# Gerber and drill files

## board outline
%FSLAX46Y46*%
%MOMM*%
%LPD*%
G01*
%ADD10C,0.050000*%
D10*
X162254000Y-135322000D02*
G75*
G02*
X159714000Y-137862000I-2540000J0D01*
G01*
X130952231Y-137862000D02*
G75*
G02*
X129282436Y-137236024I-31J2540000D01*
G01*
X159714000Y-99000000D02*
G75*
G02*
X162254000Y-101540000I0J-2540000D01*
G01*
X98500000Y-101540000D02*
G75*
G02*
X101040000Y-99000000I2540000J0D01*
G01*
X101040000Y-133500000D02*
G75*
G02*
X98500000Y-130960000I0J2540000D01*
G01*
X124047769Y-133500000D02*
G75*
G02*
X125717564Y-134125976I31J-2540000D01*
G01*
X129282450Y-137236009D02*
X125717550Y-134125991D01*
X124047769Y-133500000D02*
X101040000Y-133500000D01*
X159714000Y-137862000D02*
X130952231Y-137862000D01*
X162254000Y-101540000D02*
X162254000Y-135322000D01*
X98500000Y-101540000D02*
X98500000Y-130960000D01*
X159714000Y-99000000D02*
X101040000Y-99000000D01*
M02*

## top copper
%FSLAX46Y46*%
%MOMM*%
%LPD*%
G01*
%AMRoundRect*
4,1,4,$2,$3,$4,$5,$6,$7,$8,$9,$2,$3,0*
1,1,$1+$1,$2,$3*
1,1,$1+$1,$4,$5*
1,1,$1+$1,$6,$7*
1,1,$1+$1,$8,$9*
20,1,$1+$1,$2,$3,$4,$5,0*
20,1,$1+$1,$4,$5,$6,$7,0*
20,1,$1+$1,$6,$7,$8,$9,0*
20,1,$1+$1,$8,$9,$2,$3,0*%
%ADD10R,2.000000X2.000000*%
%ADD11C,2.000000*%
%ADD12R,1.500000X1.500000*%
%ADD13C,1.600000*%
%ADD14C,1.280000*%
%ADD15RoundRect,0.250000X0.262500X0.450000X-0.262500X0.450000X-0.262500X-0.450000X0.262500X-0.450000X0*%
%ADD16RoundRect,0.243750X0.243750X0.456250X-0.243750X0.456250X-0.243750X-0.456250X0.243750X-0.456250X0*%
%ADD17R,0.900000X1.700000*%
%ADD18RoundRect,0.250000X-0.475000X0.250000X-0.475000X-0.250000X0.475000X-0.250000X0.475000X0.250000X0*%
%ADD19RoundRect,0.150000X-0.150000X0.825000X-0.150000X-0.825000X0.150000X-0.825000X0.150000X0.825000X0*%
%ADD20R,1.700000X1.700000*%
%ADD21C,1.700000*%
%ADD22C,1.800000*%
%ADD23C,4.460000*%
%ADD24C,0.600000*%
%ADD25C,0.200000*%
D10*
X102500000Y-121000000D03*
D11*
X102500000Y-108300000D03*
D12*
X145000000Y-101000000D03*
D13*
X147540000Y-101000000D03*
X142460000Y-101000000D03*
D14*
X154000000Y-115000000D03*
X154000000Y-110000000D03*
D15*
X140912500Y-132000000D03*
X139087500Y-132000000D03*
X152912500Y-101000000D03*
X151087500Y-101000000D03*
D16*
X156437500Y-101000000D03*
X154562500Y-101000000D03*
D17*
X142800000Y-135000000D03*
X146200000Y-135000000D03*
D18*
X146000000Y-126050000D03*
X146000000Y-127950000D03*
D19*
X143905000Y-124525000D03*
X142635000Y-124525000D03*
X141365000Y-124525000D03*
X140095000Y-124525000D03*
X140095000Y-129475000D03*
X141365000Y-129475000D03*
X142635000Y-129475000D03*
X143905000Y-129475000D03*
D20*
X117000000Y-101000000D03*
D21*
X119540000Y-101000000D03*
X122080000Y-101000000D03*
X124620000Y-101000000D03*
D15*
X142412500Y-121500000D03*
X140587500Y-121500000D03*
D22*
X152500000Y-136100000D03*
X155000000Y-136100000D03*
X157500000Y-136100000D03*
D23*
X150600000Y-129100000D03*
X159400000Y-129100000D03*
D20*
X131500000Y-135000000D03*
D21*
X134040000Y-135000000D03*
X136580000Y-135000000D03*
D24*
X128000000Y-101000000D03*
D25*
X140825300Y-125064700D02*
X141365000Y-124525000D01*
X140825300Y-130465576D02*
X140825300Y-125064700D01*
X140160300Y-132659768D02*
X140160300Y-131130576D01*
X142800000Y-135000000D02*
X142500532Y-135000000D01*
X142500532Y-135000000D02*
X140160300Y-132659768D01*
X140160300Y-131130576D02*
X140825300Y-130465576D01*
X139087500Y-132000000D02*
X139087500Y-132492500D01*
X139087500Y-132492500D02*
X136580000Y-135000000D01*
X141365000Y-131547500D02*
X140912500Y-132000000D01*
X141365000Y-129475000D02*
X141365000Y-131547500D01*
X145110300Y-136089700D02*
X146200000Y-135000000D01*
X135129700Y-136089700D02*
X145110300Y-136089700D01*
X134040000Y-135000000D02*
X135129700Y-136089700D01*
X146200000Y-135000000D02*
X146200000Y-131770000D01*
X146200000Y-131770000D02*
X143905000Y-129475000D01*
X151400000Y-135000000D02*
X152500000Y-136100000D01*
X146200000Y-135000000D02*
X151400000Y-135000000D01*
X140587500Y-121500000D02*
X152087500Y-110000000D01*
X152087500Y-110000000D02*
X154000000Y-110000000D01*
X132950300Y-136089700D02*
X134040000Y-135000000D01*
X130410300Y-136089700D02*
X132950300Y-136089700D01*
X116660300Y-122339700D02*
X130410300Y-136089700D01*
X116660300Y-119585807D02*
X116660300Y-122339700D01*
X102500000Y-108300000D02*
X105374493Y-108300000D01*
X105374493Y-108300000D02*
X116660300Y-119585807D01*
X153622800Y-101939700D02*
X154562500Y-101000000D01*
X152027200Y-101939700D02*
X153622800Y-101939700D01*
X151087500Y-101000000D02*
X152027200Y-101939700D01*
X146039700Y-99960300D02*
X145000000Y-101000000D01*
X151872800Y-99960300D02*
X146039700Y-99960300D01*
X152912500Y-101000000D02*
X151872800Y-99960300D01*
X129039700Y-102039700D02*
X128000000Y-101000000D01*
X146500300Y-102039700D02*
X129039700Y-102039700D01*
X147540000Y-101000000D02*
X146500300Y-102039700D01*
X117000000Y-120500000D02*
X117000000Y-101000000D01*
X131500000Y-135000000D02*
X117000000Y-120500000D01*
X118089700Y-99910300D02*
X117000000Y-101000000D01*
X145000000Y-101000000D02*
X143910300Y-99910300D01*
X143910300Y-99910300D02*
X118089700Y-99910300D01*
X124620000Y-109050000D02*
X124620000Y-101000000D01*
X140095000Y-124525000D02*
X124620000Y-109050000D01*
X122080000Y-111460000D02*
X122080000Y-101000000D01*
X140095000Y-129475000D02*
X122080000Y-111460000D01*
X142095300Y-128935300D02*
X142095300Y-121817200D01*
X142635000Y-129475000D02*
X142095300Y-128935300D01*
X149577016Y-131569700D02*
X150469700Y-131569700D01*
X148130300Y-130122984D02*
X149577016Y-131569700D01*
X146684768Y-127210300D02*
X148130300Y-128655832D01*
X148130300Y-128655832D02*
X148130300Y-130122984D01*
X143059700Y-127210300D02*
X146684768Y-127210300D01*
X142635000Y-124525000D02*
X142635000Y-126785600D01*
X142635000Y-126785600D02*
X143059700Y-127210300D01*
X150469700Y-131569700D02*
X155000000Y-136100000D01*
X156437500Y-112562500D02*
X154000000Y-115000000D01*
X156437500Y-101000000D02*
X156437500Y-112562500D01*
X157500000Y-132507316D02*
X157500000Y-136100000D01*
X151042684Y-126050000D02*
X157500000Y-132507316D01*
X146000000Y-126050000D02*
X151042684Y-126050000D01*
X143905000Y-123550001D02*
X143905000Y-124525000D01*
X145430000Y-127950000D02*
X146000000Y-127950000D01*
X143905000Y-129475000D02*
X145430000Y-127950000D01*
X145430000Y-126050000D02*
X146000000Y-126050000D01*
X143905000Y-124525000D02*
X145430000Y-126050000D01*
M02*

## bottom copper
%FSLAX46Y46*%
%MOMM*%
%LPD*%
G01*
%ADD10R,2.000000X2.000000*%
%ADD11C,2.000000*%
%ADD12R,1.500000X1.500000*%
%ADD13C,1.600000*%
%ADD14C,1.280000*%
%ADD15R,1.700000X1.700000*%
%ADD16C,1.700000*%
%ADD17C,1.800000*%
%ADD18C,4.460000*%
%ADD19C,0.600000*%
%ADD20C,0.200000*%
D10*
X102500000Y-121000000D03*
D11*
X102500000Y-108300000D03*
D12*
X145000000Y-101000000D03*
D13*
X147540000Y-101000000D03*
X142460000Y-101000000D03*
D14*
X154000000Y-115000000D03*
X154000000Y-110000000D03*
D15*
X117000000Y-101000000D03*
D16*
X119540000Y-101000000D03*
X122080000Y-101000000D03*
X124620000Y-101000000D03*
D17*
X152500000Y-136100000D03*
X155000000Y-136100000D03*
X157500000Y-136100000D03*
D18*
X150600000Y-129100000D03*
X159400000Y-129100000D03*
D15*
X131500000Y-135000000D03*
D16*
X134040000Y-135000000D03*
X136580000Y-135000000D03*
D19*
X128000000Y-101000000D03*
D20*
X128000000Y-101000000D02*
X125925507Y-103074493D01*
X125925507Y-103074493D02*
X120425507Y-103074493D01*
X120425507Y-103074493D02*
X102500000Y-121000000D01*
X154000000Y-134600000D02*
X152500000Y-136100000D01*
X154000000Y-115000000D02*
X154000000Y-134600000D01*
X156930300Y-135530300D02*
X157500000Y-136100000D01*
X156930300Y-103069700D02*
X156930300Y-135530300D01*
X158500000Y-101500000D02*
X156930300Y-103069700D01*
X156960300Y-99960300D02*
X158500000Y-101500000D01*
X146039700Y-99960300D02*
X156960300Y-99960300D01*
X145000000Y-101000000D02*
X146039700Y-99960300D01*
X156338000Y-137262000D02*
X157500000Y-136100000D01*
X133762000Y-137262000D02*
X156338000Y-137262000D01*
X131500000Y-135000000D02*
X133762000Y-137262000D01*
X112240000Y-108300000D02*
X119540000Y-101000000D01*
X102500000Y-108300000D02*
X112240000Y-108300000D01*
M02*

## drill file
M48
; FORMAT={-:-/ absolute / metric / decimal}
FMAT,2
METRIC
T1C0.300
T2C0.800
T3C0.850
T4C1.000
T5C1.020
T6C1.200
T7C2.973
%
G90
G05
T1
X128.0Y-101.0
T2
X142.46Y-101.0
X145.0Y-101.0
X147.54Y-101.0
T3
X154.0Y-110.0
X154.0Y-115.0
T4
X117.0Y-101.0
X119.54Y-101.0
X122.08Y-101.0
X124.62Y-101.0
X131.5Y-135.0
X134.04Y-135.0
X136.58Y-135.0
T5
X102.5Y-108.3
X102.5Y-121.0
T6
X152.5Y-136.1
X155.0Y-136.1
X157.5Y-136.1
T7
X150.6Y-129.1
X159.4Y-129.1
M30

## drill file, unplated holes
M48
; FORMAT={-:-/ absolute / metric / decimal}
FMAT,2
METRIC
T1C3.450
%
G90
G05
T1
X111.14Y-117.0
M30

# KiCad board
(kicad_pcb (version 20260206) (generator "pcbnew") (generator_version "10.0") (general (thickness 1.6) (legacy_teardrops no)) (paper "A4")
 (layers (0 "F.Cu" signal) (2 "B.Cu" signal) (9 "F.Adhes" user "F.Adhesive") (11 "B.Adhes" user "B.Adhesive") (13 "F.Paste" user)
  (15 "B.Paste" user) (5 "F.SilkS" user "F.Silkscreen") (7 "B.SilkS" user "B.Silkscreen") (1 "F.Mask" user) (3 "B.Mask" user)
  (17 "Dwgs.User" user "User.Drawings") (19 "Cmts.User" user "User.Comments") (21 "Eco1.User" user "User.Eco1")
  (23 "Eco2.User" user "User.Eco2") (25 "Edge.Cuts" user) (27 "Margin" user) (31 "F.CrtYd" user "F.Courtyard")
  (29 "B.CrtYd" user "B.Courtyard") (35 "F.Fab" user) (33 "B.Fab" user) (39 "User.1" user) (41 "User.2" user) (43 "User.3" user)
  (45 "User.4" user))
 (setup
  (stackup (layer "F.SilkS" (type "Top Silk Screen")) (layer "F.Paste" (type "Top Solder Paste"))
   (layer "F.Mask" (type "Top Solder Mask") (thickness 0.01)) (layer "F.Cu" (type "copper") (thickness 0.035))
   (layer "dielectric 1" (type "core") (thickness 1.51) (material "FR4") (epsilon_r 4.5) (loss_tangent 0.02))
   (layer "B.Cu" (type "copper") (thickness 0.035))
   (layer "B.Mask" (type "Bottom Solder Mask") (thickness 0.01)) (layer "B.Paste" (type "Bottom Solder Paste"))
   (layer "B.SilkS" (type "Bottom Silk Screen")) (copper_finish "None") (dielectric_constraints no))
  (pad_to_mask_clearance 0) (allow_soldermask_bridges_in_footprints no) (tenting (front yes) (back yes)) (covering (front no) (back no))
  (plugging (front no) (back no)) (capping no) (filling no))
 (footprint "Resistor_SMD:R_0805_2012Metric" (layer "F.Cu") (at 140 132 180)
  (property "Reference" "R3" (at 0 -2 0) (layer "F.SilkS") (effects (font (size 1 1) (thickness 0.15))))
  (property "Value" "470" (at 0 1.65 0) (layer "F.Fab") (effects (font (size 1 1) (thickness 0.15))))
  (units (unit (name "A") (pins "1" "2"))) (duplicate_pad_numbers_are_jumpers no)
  (pad "1" smd roundrect (at -0.9125 0 180) (size 1.025 1.4) (layers "F.Cu" "F.Mask" "F.Paste") (roundrect_rratio 0.243902)
   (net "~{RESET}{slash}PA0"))
  (pad "2" smd roundrect (at 0.9125 0 180) (size 1.025 1.4) (layers "F.Cu" "F.Mask" "F.Paste") (roundrect_rratio 0.243902) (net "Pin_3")))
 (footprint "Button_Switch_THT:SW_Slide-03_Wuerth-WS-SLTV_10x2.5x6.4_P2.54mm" (layer "F.Cu") (at 145 101 180)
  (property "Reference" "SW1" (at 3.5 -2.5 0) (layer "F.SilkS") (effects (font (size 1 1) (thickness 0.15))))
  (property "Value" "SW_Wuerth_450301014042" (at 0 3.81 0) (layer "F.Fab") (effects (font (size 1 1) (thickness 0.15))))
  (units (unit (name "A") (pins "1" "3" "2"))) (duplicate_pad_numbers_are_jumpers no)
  (pad "1" thru_hole rect (at 0 0 180) (size 1.5 1.5) (drill 0.8) (layers "*.Cu" "*.Mask") (remove_unused_layers no) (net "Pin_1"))
  (pad "2" thru_hole circle (at -2.54 0 180) (size 1.6 1.6) (drill 0.8) (layers "*.Cu" "*.Mask") (remove_unused_layers no)
   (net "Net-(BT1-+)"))
  (pad "3" thru_hole circle (at 2.54 0 180) (size 1.6 1.6) (drill 0.8) (layers "*.Cu" "*.Mask") (remove_unused_layers no)
   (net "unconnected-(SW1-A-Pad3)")))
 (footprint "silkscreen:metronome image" (layer "F.Cu") (at 143.5 113)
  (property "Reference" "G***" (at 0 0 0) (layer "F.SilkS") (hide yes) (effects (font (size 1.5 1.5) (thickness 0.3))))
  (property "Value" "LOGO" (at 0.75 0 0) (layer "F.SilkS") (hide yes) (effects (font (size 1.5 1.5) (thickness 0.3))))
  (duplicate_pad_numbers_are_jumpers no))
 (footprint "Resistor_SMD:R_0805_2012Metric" (layer "F.Cu") (at 152 101 180)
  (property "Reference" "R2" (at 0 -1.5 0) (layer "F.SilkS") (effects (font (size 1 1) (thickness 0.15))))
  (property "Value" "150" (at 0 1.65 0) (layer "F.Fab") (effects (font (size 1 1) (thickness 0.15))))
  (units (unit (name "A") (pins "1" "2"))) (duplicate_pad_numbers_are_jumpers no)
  (pad "1" smd roundrect (at -0.9125 0 180) (size 1.025 1.4) (layers "F.Cu" "F.Mask" "F.Paste") (roundrect_rratio 0.243902) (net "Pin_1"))
  (pad "2" smd roundrect (at 0.9125 0 180) (size 1.025 1.4) (layers "F.Cu" "F.Mask" "F.Paste") (roundrect_rratio 0.243902)
   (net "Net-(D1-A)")))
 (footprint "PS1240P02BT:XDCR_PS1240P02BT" (layer "F.Cu") (at 154 112.5 -90)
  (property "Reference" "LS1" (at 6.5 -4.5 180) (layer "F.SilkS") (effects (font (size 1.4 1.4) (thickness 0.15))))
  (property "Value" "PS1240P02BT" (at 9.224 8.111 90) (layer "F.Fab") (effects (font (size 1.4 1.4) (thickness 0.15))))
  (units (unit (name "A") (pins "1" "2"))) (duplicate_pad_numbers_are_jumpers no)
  (pad "1" thru_hole circle (at -2.5 0 270) (size 1.28 1.28) (drill 0.85) (layers "*.Cu" "*.Mask") (remove_unused_layers no)
   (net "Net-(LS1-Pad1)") (solder_mask_margin 0.102))
  (pad "2" thru_hole circle (at 2.5 0 270) (size 1.28 1.28) (drill 0.85) (layers "*.Cu" "*.Mask") (remove_unused_layers no) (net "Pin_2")
   (solder_mask_margin 0.102)))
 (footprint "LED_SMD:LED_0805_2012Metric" (layer "F.Cu") (at 155.5 101 180)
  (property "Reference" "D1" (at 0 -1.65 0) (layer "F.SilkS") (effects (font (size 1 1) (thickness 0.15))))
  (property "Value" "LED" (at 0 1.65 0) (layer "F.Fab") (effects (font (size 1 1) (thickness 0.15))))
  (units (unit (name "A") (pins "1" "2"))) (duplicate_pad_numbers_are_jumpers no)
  (pad "1" smd roundrect (at -0.9375 0 180) (size 0.975 1.4) (layers "F.Cu" "F.Mask" "F.Paste") (roundrect_rratio 0.25) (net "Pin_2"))
  (pad "2" smd roundrect (at 0.9375 0 180) (size 0.975 1.4) (layers "F.Cu" "F.Mask" "F.Paste") (roundrect_rratio 0.25) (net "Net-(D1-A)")))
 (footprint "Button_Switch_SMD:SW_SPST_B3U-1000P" (layer "F.Cu") (at 144.5 135)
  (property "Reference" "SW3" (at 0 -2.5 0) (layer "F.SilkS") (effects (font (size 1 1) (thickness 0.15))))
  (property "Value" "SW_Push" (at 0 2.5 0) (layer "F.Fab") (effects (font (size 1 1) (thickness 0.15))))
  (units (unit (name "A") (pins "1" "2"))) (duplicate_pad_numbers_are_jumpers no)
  (pad "1" smd rect (at -1.7 0) (size 0.9 1.7) (layers "F.Cu" "F.Mask" "F.Paste") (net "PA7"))
  (pad "2" smd rect (at 1.7 0) (size 0.9 1.7) (layers "F.Cu" "F.Mask" "F.Paste") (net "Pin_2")))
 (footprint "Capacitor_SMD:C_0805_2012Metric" (layer "F.Cu") (at 146 127 -90)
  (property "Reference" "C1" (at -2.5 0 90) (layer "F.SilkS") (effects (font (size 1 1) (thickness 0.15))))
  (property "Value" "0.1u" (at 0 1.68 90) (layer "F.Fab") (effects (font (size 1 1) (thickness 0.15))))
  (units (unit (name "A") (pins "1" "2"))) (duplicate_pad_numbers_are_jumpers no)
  (pad "1" smd roundrect (at -0.95 0 270) (size 1 1.45) (layers "F.Cu" "F.Mask" "F.Paste") (roundrect_rratio 0.25) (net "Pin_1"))
  (pad "2" smd roundrect (at 0.95 0 270) (size 1 1.45) (layers "F.Cu" "F.Mask" "F.Paste") (roundrect_rratio 0.25) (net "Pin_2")))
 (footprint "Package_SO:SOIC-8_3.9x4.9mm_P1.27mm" (layer "F.Cu") (at 142 127 -90)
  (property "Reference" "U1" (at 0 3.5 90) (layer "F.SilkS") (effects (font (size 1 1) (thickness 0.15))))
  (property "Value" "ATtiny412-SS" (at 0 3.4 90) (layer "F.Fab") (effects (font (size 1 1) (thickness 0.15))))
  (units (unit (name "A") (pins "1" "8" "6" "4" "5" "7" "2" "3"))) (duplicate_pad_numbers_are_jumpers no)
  (pad "1" smd roundrect (at -2.475 -1.905 270) (size 1.95 0.6) (layers "F.Cu" "F.Mask" "F.Paste") (roundrect_rratio 0.25) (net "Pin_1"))
  (pad "2" smd roundrect (at -2.475 -0.635 270) (size 1.95 0.6) (layers "F.Cu" "F.Mask" "F.Paste") (roundrect_rratio 0.25) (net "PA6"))
  (pad "3" smd roundrect (at -2.475 0.635 270) (size 1.95 0.6) (layers "F.Cu" "F.Mask" "F.Paste") (roundrect_rratio 0.25) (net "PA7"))
  (pad "4" smd roundrect (at -2.475 1.905 270) (size 1.95 0.6) (layers "F.Cu" "F.Mask" "F.Paste") (roundrect_rratio 0.25) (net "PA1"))
  (pad "5" smd roundrect (at 2.475 1.905 270) (size 1.95 0.6) (layers "F.Cu" "F.Mask" "F.Paste") (roundrect_rratio 0.25) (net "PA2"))
  (pad "6" smd roundrect (at 2.475 0.635 270) (size 1.95 0.6) (layers "F.Cu" "F.Mask" "F.Paste") (roundrect_rratio 0.25)
   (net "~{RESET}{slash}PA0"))
  (pad "7" smd roundrect (at 2.475 -0.635 270) (size 1.95 0.6) (layers "F.Cu" "F.Mask" "F.Paste") (roundrect_rratio 0.25) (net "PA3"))
  (pad "8" smd roundrect (at 2.475 -1.905 270) (size 1.95 0.6) (layers "F.Cu" "F.Mask" "F.Paste") (roundrect_rratio 0.25) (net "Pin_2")))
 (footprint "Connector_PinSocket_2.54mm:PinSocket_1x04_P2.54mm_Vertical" (layer "F.Cu") (at 117 101 90)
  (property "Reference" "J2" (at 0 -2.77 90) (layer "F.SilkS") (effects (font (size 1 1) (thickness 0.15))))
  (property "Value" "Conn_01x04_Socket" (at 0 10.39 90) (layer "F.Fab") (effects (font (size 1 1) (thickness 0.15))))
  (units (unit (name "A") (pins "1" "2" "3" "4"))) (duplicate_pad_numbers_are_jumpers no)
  (pad "1" thru_hole rect (at 0 0 90) (size 1.7 1.7) (drill 1) (layers "*.Cu" "*.Mask") (remove_unused_layers no) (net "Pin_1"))
  (pad "2" thru_hole circle (at 0 2.54 90) (size 1.7 1.7) (drill 1) (layers "*.Cu" "*.Mask") (remove_unused_layers no) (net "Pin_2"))
  (pad "3" thru_hole circle (at 0 5.08 90) (size 1.7 1.7) (drill 1) (layers "*.Cu" "*.Mask") (remove_unused_layers no) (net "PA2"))
  (pad "4" thru_hole circle (at 0 7.62 90) (size 1.7 1.7) (drill 1) (layers "*.Cu" "*.Mask") (remove_unused_layers no) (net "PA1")))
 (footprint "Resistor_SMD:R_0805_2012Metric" (layer "F.Cu") (at 141.5 121.5 180)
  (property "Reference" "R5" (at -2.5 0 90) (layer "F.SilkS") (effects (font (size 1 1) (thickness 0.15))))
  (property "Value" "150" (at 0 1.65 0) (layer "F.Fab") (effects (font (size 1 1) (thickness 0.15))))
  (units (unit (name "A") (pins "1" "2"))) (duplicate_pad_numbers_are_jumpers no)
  (pad "1" smd roundrect (at -0.9125 0 180) (size 1.025 1.4) (layers "F.Cu" "F.Mask" "F.Paste") (roundrect_rratio 0.243902) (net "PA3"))
  (pad "2" smd roundrect (at 0.9125 0 180) (size 1.025 1.4) (layers "F.Cu" "F.Mask" "F.Paste") (roundrect_rratio 0.243902)
   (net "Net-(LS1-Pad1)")))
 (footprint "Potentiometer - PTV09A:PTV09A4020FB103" (layer "F.Cu") (at 155 130.5)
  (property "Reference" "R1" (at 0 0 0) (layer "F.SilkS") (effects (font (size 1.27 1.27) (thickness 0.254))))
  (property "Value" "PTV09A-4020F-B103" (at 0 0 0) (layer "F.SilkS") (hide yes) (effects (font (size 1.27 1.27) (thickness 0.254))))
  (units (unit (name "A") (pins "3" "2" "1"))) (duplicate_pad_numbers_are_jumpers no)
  (pad "1" thru_hole circle (at -2.5 5.6) (size 1.8 1.8) (drill 1.2) (layers "*.Cu" "*.Mask") (remove_unused_layers no) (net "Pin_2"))
  (pad "2" thru_hole circle (at 0 5.6) (size 1.8 1.8) (drill 1.2) (layers "*.Cu" "*.Mask") (remove_unused_layers no) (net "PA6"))
  (pad "3" thru_hole circle (at 2.5 5.6) (size 1.8 1.8) (drill 1.2) (layers "*.Cu" "*.Mask") (remove_unused_layers no) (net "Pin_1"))
  (pad "4" thru_hole circle (at -4.4 -1.4) (size 4.46 4.46) (drill 2.9732) (layers "*.Cu" "*.Mask") (remove_unused_layers no))
  (pad "5" thru_hole circle (at 4.4 -1.4) (size 4.46 4.46) (drill 2.9732) (layers "*.Cu" "*.Mask") (remove_unused_layers no)))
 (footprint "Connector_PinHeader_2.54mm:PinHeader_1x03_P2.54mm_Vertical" (layer "F.Cu") (at 131.5 135 90)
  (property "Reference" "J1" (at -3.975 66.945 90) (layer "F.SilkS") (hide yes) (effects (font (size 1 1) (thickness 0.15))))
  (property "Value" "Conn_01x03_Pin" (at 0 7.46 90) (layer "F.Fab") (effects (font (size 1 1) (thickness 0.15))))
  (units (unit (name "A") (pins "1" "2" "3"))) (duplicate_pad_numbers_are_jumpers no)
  (pad "1" thru_hole rect (at 0 0 90) (size 1.7 1.7) (drill 1) (layers "*.Cu" "*.Mask") (remove_unused_layers no) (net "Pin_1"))
  (pad "2" thru_hole circle (at 0 2.54 90) (size 1.7 1.7) (drill 1) (layers "*.Cu" "*.Mask") (remove_unused_layers no) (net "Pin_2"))
  (pad "3" thru_hole circle (at 0 5.08 90) (size 1.7 1.7) (drill 1) (layers "*.Cu" "*.Mask") (remove_unused_layers no) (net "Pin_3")))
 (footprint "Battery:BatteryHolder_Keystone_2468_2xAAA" (layer "B.Cu") (at 102.5 121)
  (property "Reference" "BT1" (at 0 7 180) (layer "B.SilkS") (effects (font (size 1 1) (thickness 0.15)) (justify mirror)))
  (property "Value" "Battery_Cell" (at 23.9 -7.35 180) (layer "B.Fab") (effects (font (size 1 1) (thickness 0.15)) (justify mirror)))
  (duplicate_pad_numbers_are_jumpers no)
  (pad "" np_thru_hole circle (at 8.64 -4) (size 3.45 3.45) (drill 3.45) (layers "*.Cu"))
  (pad "1" thru_hole rect (at 0 0) (size 2 2) (drill 1.02) (layers "*.Cu" "*.Mask") (remove_unused_layers no) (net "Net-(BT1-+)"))
  (pad "2" thru_hole circle (at 0 -12.7) (size 2 2) (drill 1.02) (layers "*.Cu" "*.Mask") (remove_unused_layers no) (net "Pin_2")))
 (gr_line (start 98.5 101.54) (end 98.5 130.96) (stroke (width 0.05) (type default)) (layer "Edge.Cuts"))
 (gr_arc (start 98.5 101.54) (mid 99.243949 99.743949) (end 101.04 99) (stroke (width 0.05) (type default)) (layer "Edge.Cuts"))
 (gr_arc (start 101.04 133.5) (mid 99.243949 132.756051) (end 98.5 130.96) (stroke (width 0.05) (type default)) (layer "Edge.Cuts"))
 (gr_line (start 124.047769 133.5) (end 101.04 133.5) (stroke (width 0.05) (type default)) (layer "Edge.Cuts"))
 (gr_arc (start 124.047769 133.5) (mid 124.939401 133.661641) (end 125.71755 134.125991) (stroke (width 0.05) (type default))
  (layer "Edge.Cuts"))
 (gr_line (start 129.28245 137.236009) (end 125.71755 134.125991) (stroke (width 0.05) (type default)) (layer "Edge.Cuts"))
 (gr_arc (start 130.952231 137.862) (mid 130.060599 137.700359) (end 129.28245 137.236009) (stroke (width 0.05) (type default))
  (layer "Edge.Cuts"))
 (gr_line (start 159.714 99) (end 101.04 99) (stroke (width 0.05) (type default)) (layer "Edge.Cuts"))
 (gr_arc (start 159.714 99) (mid 161.510051 99.743949) (end 162.254 101.54) (stroke (width 0.05) (type default)) (layer "Edge.Cuts"))
 (gr_line (start 159.714 137.862) (end 130.952231 137.862) (stroke (width 0.05) (type default)) (layer "Edge.Cuts"))
 (gr_line (start 162.254 101.54) (end 162.254 135.322) (stroke (width 0.05) (type default)) (layer "Edge.Cuts"))
 (gr_arc (start 162.254 135.322) (mid 161.510051 137.118051) (end 159.714 137.862) (stroke (width 0.05) (type default)) (layer "Edge.Cuts"))
 (segment (start 141.365 131.5475) (end 140.9125 132) (width 0.2) (layer "F.Cu") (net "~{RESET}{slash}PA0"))
 (segment (start 141.365 129.475) (end 141.365 131.5475) (width 0.2) (layer "F.Cu") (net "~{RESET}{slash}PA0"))
 (segment (start 139.0875 132.4925) (end 136.58 135) (width 0.2) (layer "F.Cu") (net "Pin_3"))
 (segment (start 139.0875 132) (end 139.0875 132.4925) (width 0.2) (layer "F.Cu") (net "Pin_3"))
 (segment (start 146 126.05) (end 151.042684 126.05) (width 0.2) (layer "F.Cu") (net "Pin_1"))
 (segment (start 151.8728 99.9603) (end 146.0397 99.9603) (width 0.2) (layer "F.Cu") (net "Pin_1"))
 (segment (start 143.9103 99.9103) (end 118.0897 99.9103) (width 0.2) (layer "F.Cu") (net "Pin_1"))
 (segment (start 145.43 126.05) (end 146 126.05) (width 0.2) (layer "F.Cu") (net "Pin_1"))
 (segment (start 131.5 135) (end 117 120.5) (width 0.2) (layer "F.Cu") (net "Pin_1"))
 (segment (start 145 101) (end 143.9103 99.9103) (width 0.2) (layer "F.Cu") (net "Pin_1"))
 (segment (start 146.0397 99.9603) (end 145 101) (width 0.2) (layer "F.Cu") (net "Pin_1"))
 (segment (start 151.042684 126.05) (end 157.5 132.507316) (width 0.2) (layer "F.Cu") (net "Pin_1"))
 (segment (start 117 120.5) (end 117 101) (width 0.2) (layer "F.Cu") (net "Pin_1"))
 (segment (start 143.905 124.525) (end 145.43 126.05) (width 0.2) (layer "F.Cu") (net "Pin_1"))
 (segment (start 143.905 123.550001) (end 143.905 124.525) (width 0.2) (layer "F.Cu") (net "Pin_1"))
 (segment (start 118.0897 99.9103) (end 117 101) (width 0.2) (layer "F.Cu") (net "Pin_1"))
 (segment (start 152.9125 101) (end 151.8728 99.9603) (width 0.2) (layer "F.Cu") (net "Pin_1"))
 (segment (start 157.5 132.507316) (end 157.5 136.1) (width 0.2) (layer "F.Cu") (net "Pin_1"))
 (segment (start 133.762 137.262) (end 156.338 137.262) (width 0.2) (layer "B.Cu") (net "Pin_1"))
 (segment (start 156.9303 103.0697) (end 156.9303 135.5303) (width 0.2) (layer "B.Cu") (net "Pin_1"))
 (segment (start 145 101) (end 146.0397 99.9603) (width 0.2) (layer "B.Cu") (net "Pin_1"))
 (segment (start 146.0397 99.9603) (end 156.9603 99.9603) (width 0.2) (layer "B.Cu") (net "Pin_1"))
 (segment (start 158.5 101.5) (end 156.9303 103.0697) (width 0.2) (layer "B.Cu") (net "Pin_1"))
 (segment (start 156.9303 135.5303) (end 157.5 136.1) (width 0.2) (layer "B.Cu") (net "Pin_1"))
 (segment (start 131.5 135) (end 133.762 137.262) (width 0.2) (layer "B.Cu") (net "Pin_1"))
 (segment (start 156.9603 99.9603) (end 158.5 101.5) (width 0.2) (layer "B.Cu") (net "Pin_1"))
 (segment (start 156.338 137.262) (end 157.5 136.1) (width 0.2) (layer "B.Cu") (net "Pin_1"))
 (segment (start 146.5003 102.0397) (end 129.0397 102.0397) (width 0.2) (layer "F.Cu") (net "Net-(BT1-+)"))
 (segment (start 129.0397 102.0397) (end 128 101) (width 0.2) (layer "F.Cu") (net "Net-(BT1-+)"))
 (segment (start 147.54 101) (end 146.5003 102.0397) (width 0.2) (layer "F.Cu") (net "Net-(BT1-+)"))
 (via (at 128 101) (size 0.6) (drill 0.3) (layers "F.Cu" "B.Cu") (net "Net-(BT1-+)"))
 (segment (start 128 101) (end 125.925507 103.074493) (width 0.2) (layer "B.Cu") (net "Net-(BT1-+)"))
 (segment (start 120.425507 103.074493) (end 102.5 121) (width 0.2) (layer "B.Cu") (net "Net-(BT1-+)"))
 (segment (start 125.925507 103.074493) (end 120.425507 103.074493) (width 0.2) (layer "B.Cu") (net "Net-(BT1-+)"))
 (segment (start 153.6228 101.9397) (end 154.5625 101) (width 0.2) (layer "F.Cu") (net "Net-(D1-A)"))
 (segment (start 152.0272 101.9397) (end 153.6228 101.9397) (width 0.2) (layer "F.Cu") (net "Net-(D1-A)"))
 (segment (start 151.0875 101) (end 152.0272 101.9397) (width 0.2) (layer "F.Cu") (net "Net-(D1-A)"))
 (segment (start 152.0875 110) (end 154 110) (width 0.2) (layer "F.Cu") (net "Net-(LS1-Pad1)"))
 (segment (start 140.5875 121.5) (end 152.0875 110) (width 0.2) (layer "F.Cu") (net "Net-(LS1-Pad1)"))
 (segment (start 146.2 131.77) (end 143.905 129.475) (width 0.2) (layer "F.Cu") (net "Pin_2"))
 (segment (start 132.9503 136.0897) (end 134.04 135) (width 0.2) (layer "F.Cu") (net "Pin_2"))
 (segment (start 116.6603 119.585807) (end 116.6603 122.3397) (width 0.2) (layer "F.Cu") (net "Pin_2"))
 (segment (start 135.1297 136.0897) (end 145.1103 136.0897) (width 0.2) (layer "F.Cu") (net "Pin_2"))
 (segment (start 146.2 135) (end 151.4 135) (width 0.2) (layer "F.Cu") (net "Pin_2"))
 (segment (start 145.43 127.95) (end 146 127.95) (width 0.2) (layer "F.Cu") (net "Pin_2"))
 (segment (start 146.2 135) (end 146.2 131.77) (width 0.2) (layer "F.Cu") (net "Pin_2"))
 (segment (start 130.4103 136.0897) (end 132.9503 136.0897) (width 0.2) (layer "F.Cu") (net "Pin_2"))
 (segment (start 156.4375 112.5625) (end 154 115) (width 0.2) (layer "F.Cu") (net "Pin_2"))
 (segment (start 102.5 108.3) (end 105.374493 108.3) (width 0.2) (layer "F.Cu") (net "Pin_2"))
 (segment (start 145.1103 136.0897) (end 146.2 135) (width 0.2) (layer "F.Cu") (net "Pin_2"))
 (segment (start 116.6603 122.3397) (end 130.4103 136.0897) (width 0.2) (layer "F.Cu") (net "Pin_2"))
 (segment (start 105.374493 108.3) (end 116.6603 119.585807) (width 0.2) (layer "F.Cu") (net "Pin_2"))
 (segment (start 156.4375 101) (end 156.4375 112.5625) (width 0.2) (layer "F.Cu") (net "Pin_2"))
 (segment (start 143.905 129.475) (end 145.43 127.95) (width 0.2) (layer "F.Cu") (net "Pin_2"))
 (segment (start 151.4 135) (end 152.5 136.1) (width 0.2) (layer "F.Cu") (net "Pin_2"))
 (segment (start 134.04 135) (end 135.1297 136.0897) (width 0.2) (layer "F.Cu") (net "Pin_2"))
 (segment (start 154 115) (end 154 134.6) (width 0.2) (layer "B.Cu") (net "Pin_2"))
 (segment (start 102.5 108.3) (end 112.24 108.3) (width 0.2) (layer "B.Cu") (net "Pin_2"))
 (segment (start 112.24 108.3) (end 119.54 101) (width 0.2) (layer "B.Cu") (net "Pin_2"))
 (segment (start 154 134.6) (end 152.5 136.1) (width 0.2) (layer "B.Cu") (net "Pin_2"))
 (segment (start 140.8253 125.0647) (end 141.365 124.525) (width 0.2) (layer "F.Cu") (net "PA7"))
 (segment (start 140.8253 130.465576) (end 140.8253 125.0647) (width 0.2) (layer "F.Cu") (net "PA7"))
 (segment (start 140.1603 131.130576) (end 140.8253 130.465576) (width 0.2) (layer "F.Cu") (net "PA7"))
 (segment (start 142.8 135) (end 142.500532 135) (width 0.2) (layer "F.Cu") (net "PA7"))
 (segment (start 142.500532 135) (end 140.1603 132.659768) (width 0.2) (layer "F.Cu") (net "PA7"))
 (segment (start 140.1603 132.659768) (end 140.1603 131.130576) (width 0.2) (layer "F.Cu") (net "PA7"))
 (segment (start 142.635 124.525) (end 142.635 126.7856) (width 0.2) (layer "F.Cu") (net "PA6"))
 (segment (start 146.684768 127.2103) (end 148.1303 128.655832) (width 0.2) (layer "F.Cu") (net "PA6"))
 (segment (start 148.1303 128.655832) (end 148.1303 130.122984) (width 0.2) (layer "F.Cu") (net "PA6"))
 (segment (start 142.635 126.7856) (end 143.0597 127.2103) (width 0.2) (layer "F.Cu") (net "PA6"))
 (segment (start 149.577016 131.5697) (end 150.4697 131.5697) (width 0.2) (layer "F.Cu") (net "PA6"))
 (segment (start 150.4697 131.5697) (end 155 136.1) (width 0.2) (layer "F.Cu") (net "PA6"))
 (segment (start 143.0597 127.2103) (end 146.684768 127.2103) (width 0.2) (layer "F.Cu") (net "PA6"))
 (segment (start 148.1303 130.122984) (end 149.577016 131.5697) (width 0.2) (layer "F.Cu") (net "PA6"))
 (segment (start 140.095 124.525) (end 124.62 109.05) (width 0.2) (layer "F.Cu") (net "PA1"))
 (segment (start 124.62 109.05) (end 124.62 101) (width 0.2) (layer "F.Cu") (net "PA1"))
 (segment (start 140.095 129.475) (end 122.08 111.46) (width 0.2) (layer "F.Cu") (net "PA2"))
 (segment (start 122.08 111.46) (end 122.08 101) (width 0.2) (layer "F.Cu") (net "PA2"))
 (segment (start 142.635 129.475) (end 142.0953 128.9353) (width 0.2) (layer "F.Cu") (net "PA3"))
 (segment (start 142.0953 128.9353) (end 142.0953 121.8172) (width 0.2) (layer "F.Cu") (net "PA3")))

